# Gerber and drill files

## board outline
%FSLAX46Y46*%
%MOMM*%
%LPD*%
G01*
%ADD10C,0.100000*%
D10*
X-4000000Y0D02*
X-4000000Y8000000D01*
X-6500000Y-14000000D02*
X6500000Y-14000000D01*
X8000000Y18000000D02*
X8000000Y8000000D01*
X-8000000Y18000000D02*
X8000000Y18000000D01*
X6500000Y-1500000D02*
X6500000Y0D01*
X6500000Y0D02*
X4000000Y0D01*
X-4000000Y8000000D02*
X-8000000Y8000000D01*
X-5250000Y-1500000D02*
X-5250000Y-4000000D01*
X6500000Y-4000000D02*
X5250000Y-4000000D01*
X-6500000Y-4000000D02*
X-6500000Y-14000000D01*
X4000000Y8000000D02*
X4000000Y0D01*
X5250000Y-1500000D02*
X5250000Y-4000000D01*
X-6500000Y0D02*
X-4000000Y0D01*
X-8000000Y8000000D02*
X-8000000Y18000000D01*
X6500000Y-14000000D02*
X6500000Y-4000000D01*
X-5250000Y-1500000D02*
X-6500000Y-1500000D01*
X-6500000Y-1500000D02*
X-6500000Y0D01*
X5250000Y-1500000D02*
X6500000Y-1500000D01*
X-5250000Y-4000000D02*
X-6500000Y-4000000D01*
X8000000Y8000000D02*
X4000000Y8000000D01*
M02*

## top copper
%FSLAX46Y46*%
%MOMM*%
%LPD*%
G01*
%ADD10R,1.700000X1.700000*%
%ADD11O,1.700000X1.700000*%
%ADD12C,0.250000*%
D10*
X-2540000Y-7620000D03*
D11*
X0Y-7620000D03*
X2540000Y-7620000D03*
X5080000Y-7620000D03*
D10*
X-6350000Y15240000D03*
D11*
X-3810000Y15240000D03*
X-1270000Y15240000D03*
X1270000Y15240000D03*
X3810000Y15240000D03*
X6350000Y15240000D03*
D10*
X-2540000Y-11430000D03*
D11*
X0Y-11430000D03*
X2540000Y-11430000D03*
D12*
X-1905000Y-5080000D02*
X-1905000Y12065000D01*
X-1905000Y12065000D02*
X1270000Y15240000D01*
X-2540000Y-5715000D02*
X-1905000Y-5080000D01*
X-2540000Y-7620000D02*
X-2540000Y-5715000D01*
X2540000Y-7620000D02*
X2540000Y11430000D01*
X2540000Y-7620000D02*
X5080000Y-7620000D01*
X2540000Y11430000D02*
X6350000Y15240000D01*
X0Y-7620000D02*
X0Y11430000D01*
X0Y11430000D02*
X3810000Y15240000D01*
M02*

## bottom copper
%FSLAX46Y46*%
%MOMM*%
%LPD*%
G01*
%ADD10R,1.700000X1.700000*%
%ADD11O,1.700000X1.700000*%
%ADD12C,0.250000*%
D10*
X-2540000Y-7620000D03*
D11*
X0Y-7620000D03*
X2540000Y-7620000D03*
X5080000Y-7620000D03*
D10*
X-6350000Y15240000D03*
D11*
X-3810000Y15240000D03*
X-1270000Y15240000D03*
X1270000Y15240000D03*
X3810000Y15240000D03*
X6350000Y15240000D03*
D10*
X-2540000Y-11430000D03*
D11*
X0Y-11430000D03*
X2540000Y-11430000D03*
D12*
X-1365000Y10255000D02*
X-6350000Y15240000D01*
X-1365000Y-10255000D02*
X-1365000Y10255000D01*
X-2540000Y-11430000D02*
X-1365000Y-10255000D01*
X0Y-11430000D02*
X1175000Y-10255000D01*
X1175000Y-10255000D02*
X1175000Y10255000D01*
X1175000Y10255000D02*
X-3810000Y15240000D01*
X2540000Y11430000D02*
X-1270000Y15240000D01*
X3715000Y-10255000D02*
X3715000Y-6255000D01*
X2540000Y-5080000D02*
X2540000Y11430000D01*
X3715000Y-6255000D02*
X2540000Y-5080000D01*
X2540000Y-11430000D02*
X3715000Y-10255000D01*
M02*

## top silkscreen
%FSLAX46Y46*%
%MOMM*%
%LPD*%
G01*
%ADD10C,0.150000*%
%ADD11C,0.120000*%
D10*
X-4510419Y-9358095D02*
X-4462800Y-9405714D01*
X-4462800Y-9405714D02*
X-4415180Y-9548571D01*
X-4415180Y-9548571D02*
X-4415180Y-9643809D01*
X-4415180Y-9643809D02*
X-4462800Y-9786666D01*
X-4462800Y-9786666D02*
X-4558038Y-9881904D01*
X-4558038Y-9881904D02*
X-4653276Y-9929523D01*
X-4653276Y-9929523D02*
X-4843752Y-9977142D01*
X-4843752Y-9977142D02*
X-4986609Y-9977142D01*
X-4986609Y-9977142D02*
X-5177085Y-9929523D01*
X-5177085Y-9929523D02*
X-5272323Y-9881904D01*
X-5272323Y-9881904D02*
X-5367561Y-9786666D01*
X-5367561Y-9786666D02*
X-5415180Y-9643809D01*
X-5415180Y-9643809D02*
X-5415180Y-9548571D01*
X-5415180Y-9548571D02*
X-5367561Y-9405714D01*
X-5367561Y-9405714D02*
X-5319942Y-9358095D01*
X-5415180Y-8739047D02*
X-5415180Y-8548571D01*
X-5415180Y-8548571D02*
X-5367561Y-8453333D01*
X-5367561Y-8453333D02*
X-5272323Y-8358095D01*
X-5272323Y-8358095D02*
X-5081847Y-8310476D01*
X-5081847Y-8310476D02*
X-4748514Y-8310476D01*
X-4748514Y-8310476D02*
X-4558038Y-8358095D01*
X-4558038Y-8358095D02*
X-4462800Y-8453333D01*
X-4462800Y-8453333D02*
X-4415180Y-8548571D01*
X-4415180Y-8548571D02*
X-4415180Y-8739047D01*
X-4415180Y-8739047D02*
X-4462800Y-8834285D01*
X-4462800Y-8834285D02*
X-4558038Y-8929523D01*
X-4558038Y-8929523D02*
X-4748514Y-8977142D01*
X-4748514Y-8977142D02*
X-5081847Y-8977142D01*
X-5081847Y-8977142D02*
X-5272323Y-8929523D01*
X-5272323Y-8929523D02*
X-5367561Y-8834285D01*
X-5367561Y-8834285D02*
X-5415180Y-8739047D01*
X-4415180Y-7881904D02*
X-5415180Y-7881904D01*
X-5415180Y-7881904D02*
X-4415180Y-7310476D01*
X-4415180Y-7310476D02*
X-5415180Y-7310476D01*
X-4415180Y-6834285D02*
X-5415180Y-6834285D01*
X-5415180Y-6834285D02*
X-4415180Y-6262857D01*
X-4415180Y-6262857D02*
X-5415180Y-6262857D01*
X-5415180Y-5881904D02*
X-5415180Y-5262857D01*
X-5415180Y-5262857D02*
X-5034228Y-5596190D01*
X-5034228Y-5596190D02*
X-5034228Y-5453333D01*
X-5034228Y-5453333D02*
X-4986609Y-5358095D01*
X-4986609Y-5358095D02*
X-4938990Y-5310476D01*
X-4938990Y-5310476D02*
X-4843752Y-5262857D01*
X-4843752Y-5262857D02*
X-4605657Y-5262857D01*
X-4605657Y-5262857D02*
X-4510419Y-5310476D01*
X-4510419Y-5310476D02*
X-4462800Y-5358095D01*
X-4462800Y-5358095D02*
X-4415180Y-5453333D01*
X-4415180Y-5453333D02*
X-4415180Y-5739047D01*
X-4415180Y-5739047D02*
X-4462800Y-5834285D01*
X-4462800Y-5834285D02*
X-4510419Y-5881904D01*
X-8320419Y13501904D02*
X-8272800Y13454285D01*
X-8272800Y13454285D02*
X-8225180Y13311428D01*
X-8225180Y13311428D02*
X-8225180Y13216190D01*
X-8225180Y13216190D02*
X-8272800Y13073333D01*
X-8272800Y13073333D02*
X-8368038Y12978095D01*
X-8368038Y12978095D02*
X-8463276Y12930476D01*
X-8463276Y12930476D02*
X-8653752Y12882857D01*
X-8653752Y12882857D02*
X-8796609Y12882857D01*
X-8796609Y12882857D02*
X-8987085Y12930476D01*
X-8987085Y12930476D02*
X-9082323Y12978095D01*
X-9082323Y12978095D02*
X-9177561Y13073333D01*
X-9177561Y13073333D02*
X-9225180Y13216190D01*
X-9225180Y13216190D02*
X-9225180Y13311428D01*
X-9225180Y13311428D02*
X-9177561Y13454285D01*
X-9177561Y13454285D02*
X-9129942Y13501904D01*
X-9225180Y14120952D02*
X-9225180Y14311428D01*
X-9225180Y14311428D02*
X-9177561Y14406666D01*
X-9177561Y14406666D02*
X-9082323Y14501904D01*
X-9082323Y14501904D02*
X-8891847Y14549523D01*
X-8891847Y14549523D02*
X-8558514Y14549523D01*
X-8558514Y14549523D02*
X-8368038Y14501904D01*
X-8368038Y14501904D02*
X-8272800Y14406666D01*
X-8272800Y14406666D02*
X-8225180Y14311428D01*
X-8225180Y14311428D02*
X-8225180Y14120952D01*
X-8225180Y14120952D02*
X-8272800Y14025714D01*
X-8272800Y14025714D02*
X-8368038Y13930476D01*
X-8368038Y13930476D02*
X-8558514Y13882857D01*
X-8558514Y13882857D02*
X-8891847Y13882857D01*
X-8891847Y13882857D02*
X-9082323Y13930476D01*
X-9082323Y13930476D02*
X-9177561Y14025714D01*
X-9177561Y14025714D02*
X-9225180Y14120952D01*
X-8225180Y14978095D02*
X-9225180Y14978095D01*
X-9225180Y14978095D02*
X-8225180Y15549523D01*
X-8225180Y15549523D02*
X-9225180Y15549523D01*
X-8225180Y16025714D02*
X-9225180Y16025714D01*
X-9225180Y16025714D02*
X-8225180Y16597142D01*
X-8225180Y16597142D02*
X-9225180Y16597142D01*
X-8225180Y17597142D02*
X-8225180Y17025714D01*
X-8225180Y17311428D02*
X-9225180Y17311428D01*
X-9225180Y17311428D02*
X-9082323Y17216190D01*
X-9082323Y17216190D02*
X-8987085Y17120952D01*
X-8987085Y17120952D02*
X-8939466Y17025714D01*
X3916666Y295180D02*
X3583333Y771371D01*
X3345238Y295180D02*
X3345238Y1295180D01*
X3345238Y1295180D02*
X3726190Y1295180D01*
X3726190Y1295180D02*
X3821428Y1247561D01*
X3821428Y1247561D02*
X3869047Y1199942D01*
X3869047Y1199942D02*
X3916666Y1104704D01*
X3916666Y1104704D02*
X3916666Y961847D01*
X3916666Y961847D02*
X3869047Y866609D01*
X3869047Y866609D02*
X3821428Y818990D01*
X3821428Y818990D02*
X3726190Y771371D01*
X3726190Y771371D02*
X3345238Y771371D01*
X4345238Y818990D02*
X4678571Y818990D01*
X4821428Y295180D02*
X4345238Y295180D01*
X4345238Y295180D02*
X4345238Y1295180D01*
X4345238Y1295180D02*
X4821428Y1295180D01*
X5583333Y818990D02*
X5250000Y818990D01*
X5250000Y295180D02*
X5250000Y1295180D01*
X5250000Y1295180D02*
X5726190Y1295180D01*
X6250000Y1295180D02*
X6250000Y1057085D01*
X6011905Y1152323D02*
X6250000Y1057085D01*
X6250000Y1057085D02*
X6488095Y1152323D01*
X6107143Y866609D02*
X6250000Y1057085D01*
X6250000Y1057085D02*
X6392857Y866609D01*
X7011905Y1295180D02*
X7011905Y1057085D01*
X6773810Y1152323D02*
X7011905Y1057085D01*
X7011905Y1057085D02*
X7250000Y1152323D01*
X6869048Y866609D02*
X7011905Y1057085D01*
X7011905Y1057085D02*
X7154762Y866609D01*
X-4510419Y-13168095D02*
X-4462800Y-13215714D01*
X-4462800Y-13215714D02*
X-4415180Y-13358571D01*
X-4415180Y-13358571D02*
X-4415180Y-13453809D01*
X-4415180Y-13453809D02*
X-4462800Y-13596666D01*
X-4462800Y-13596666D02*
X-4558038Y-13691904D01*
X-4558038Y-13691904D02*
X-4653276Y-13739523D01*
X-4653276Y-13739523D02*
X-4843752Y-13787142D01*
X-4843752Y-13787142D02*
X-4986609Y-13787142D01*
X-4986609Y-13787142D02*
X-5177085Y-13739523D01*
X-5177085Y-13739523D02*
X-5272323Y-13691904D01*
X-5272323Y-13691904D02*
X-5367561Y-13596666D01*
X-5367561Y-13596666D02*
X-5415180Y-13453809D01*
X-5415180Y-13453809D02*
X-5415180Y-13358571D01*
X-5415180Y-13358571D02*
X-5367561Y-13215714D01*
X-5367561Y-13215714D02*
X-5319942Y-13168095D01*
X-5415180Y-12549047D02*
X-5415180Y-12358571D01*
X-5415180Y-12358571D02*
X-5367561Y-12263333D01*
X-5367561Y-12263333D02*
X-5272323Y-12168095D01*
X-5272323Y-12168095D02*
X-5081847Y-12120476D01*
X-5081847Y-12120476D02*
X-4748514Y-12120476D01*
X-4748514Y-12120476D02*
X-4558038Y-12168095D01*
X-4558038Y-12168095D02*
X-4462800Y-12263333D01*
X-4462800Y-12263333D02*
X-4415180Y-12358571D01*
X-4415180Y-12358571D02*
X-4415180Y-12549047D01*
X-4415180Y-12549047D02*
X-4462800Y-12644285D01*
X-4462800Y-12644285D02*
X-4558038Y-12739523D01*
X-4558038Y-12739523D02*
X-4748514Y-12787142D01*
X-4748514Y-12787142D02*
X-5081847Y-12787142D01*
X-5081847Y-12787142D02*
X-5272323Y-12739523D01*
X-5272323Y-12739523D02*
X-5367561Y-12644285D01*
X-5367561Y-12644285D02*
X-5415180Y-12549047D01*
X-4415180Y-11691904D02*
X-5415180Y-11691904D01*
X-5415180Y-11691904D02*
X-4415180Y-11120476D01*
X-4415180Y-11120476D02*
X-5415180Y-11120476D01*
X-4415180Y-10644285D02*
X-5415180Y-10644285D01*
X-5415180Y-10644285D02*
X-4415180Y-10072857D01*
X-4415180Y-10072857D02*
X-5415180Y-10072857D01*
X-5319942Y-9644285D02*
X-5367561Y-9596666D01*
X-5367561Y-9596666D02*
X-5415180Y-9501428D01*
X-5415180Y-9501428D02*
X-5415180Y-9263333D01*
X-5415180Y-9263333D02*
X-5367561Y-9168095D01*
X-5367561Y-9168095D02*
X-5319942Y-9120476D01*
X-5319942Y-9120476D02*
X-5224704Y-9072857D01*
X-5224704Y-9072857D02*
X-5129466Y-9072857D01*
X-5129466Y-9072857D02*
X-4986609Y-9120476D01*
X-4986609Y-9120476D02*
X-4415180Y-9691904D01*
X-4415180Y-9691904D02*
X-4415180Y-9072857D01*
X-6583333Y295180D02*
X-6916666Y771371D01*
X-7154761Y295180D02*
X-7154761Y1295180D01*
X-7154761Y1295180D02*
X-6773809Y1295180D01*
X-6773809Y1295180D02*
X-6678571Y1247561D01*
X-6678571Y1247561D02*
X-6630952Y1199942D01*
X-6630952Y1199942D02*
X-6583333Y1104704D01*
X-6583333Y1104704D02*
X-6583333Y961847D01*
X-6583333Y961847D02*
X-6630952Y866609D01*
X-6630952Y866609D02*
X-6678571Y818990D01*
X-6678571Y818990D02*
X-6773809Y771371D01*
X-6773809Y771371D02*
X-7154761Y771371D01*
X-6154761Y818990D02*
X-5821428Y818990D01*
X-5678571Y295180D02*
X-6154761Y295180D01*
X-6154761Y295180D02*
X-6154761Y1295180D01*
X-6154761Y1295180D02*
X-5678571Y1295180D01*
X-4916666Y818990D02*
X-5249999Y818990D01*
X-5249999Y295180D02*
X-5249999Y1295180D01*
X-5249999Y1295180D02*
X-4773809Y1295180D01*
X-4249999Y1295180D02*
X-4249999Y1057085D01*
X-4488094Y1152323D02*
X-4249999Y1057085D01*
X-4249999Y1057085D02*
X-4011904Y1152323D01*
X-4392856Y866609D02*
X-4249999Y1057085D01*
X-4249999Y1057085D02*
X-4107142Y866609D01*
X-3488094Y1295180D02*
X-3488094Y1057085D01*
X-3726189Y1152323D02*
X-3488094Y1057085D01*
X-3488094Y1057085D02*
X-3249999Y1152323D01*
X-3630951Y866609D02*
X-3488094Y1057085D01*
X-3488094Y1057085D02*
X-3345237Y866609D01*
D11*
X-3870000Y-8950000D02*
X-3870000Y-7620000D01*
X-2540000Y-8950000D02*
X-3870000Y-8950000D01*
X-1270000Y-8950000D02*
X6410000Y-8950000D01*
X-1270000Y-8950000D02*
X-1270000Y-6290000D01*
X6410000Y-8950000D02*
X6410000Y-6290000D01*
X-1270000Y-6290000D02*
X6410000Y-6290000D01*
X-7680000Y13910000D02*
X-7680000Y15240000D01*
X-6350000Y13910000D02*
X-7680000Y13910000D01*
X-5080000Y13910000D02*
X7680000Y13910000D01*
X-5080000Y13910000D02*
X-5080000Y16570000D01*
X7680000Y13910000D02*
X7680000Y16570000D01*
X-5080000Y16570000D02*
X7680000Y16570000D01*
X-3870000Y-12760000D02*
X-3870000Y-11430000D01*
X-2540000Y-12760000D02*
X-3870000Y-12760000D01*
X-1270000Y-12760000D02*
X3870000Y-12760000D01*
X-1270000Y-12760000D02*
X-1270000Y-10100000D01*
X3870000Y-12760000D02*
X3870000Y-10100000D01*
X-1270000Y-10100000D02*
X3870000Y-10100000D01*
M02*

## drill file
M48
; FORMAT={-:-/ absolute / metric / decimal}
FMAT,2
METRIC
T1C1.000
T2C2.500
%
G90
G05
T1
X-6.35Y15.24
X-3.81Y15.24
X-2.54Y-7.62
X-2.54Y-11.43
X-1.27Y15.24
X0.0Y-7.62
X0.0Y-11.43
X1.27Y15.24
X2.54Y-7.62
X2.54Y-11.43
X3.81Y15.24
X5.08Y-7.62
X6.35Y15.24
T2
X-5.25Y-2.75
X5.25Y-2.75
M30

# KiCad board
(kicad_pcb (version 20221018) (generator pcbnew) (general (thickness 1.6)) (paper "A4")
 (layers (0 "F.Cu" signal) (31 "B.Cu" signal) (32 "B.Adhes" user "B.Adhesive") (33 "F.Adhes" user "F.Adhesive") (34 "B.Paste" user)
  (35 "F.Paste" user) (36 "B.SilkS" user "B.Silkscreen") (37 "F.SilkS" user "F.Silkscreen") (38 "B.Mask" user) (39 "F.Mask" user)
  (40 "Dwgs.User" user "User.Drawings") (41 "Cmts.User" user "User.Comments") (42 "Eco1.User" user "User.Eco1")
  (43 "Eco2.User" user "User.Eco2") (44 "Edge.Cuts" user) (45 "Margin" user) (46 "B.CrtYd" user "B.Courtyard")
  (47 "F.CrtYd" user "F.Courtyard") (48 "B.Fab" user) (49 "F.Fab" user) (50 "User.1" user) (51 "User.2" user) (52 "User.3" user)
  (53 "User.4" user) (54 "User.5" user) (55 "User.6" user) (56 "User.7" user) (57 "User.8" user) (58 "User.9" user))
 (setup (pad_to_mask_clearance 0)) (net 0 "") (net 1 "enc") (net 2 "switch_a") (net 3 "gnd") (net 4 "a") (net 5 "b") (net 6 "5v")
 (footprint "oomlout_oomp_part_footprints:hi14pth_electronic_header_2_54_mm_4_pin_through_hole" (layer "F.Cu") (at -2.54 7.62 90)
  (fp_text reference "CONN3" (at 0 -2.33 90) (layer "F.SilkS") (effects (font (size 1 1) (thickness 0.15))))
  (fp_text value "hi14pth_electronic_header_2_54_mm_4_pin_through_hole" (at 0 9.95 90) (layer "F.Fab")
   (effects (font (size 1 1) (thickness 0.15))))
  (fp_line (start -1.33 -1.33) (end 0 -1.33) (stroke (width 0.12) (type solid)) (layer "F.SilkS"))
  (fp_line (start -1.33 0) (end -1.33 -1.33) (stroke (width 0.12) (type solid)) (layer "F.SilkS"))
  (fp_line (start -1.33 1.27) (end -1.33 8.95) (stroke (width 0.12) (type solid)) (layer "F.SilkS"))
  (fp_line (start -1.33 1.27) (end 1.33 1.27) (stroke (width 0.12) (type solid)) (layer "F.SilkS"))
  (fp_line (start -1.33 8.95) (end 1.33 8.95) (stroke (width 0.12) (type solid)) (layer "F.SilkS"))
  (fp_line (start 1.33 1.27) (end 1.33 8.95) (stroke (width 0.12) (type solid)) (layer "F.SilkS"))
  (pad "1" thru_hole rect (at 0 0 90) (size 1.7 1.7) (drill 1) (layers "*.Cu" "*.Mask") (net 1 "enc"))
  (pad "2" thru_hole oval (at 0 2.54 90) (size 1.7 1.7) (drill 1) (layers "*.Cu" "*.Mask") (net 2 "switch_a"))
  (pad "3" thru_hole oval (at 0 5.08 90) (size 1.7 1.7) (drill 1) (layers "*.Cu" "*.Mask") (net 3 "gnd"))
  (pad "4" thru_hole oval (at 0 7.62 90) (size 1.7 1.7) (drill 1) (layers "*.Cu" "*.Mask") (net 3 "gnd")))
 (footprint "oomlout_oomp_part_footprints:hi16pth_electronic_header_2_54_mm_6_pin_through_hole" (layer "F.Cu") (at -6.35 -15.24 90)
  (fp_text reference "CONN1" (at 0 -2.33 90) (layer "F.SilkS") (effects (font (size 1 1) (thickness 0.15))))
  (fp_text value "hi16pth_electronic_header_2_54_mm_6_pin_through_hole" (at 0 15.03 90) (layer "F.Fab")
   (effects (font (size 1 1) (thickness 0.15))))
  (fp_line (start -1.33 -1.33) (end 0 -1.33) (stroke (width 0.12) (type solid)) (layer "F.SilkS"))
  (fp_line (start -1.33 0) (end -1.33 -1.33) (stroke (width 0.12) (type solid)) (layer "F.SilkS"))
  (fp_line (start -1.33 1.27) (end -1.33 14.03) (stroke (width 0.12) (type solid)) (layer "F.SilkS"))
  (fp_line (start -1.33 1.27) (end 1.33 1.27) (stroke (width 0.12) (type solid)) (layer "F.SilkS"))
  (fp_line (start -1.33 14.03) (end 1.33 14.03) (stroke (width 0.12) (type solid)) (layer "F.SilkS"))
  (fp_line (start 1.33 1.27) (end 1.33 14.03) (stroke (width 0.12) (type solid)) (layer "F.SilkS"))
  (pad "1" thru_hole rect (at 0 0 90) (size 1.7 1.7) (drill 1) (layers "*.Cu" "*.Mask") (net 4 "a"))
  (pad "2" thru_hole oval (at 0 2.54 90) (size 1.7 1.7) (drill 1) (layers "*.Cu" "*.Mask") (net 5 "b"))
  (pad "3" thru_hole oval (at 0 5.08 90) (size 1.7 1.7) (drill 1) (layers "*.Cu" "*.Mask") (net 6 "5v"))
  (pad "4" thru_hole oval (at 0 7.62 90) (size 1.7 1.7) (drill 1) (layers "*.Cu" "*.Mask") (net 1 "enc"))
  (pad "5" thru_hole oval (at 0 10.16 90) (size 1.7 1.7) (drill 1) (layers "*.Cu" "*.Mask") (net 2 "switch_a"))
  (pad "6" thru_hole oval (at 0 12.7 90) (size 1.7 1.7) (drill 1) (layers "*.Cu" "*.Mask") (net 3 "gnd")))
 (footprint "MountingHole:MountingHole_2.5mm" (layer "F.Cu") (at 5.25 2.75)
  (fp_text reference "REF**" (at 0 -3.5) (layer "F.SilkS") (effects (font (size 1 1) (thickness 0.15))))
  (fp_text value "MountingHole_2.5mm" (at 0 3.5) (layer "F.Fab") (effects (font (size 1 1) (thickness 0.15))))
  (pad "" np_thru_hole circle (at 0 0) (size 2.5 2.5) (drill 2.5) (layers "*.Cu" "*.Mask")))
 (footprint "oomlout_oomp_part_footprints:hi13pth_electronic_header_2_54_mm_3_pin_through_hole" (layer "F.Cu") (at -2.54 11.43 90)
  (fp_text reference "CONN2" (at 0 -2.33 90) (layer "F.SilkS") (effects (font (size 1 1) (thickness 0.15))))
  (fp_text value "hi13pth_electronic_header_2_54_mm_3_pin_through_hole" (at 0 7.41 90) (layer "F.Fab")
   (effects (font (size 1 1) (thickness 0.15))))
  (fp_line (start -1.33 -1.33) (end 0 -1.33) (stroke (width 0.12) (type solid)) (layer "F.SilkS"))
  (fp_line (start -1.33 0) (end -1.33 -1.33) (stroke (width 0.12) (type solid)) (layer "F.SilkS"))
  (fp_line (start -1.33 1.27) (end -1.33 6.41) (stroke (width 0.12) (type solid)) (layer "F.SilkS"))
  (fp_line (start -1.33 1.27) (end 1.33 1.27) (stroke (width 0.12) (type solid)) (layer "F.SilkS"))
  (fp_line (start -1.33 6.41) (end 1.33 6.41) (stroke (width 0.12) (type solid)) (layer "F.SilkS"))
  (fp_line (start 1.33 1.27) (end 1.33 6.41) (stroke (width 0.12) (type solid)) (layer "F.SilkS"))
  (pad "1" thru_hole rect (at 0 0 90) (size 1.7 1.7) (drill 1) (layers "*.Cu" "*.Mask") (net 4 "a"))
  (pad "2" thru_hole oval (at 0 2.54 90) (size 1.7 1.7) (drill 1) (layers "*.Cu" "*.Mask") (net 5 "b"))
  (pad "3" thru_hole oval (at 0 5.08 90) (size 1.7 1.7) (drill 1) (layers "*.Cu" "*.Mask") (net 6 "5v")))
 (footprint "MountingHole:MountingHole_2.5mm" (layer "F.Cu") (at -5.25 2.75)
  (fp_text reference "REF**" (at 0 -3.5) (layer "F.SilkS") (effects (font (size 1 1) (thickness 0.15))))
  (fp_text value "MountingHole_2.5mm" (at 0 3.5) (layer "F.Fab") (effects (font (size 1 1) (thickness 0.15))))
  (pad "" np_thru_hole circle (at 0 0) (size 2.5 2.5) (drill 2.5) (layers "F&B.Cu" "*.Mask")))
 (gr_line (start -4 0) (end -4 -8) (stroke (width 0.1) (type default)) (layer "Edge.Cuts"))
 (gr_line (start -6.5 14) (end 6.5 14) (stroke (width 0.1) (type default)) (layer "Edge.Cuts"))
 (gr_line (start 8 -18) (end 8 -8) (stroke (width 0.1) (type default)) (layer "Edge.Cuts"))
 (gr_line (start -8 -18) (end 8 -18) (stroke (width 0.1) (type default)) (layer "Edge.Cuts"))
 (gr_line (start 6.5 1.5) (end 6.5 0) (stroke (width 0.1) (type default)) (layer "Edge.Cuts"))
 (gr_line (start 6.5 0) (end 4 0) (stroke (width 0.1) (type default)) (layer "Edge.Cuts"))
 (gr_line (start -4 -8) (end -8 -8) (stroke (width 0.1) (type default)) (layer "Edge.Cuts"))
 (gr_line (start -5.25 1.5) (end -5.25 4) (stroke (width 0.1) (type default)) (layer "Edge.Cuts"))
 (gr_line (start 6.5 4) (end 5.25 4) (stroke (width 0.1) (type default)) (layer "Edge.Cuts"))
 (gr_line (start -6.5 4) (end -6.5 14) (stroke (width 0.1) (type default)) (layer "Edge.Cuts"))
 (gr_line (start 4 -8) (end 4 0) (stroke (width 0.1) (type default)) (layer "Edge.Cuts"))
 (gr_line (start 5.25 1.5) (end 5.25 4) (stroke (width 0.1) (type default)) (layer "Edge.Cuts"))
 (gr_line (start -6.5 0) (end -4 0) (stroke (width 0.1) (type default)) (layer "Edge.Cuts"))
 (gr_line (start -8 -8) (end -8 -18) (stroke (width 0.1) (type default)) (layer "Edge.Cuts"))
 (gr_line (start 6.5 14) (end 6.5 4) (stroke (width 0.1) (type default)) (layer "Edge.Cuts"))
 (gr_line (start -5.25 1.5) (end -6.5 1.5) (stroke (width 0.1) (type default)) (layer "Edge.Cuts"))
 (gr_line (start -6.5 1.5) (end -6.5 0) (stroke (width 0.1) (type default)) (layer "Edge.Cuts"))
 (gr_line (start 5.25 1.5) (end 6.5 1.5) (stroke (width 0.1) (type default)) (layer "Edge.Cuts"))
 (gr_line (start -5.25 4) (end -6.5 4) (stroke (width 0.1) (type default)) (layer "Edge.Cuts"))
 (gr_line (start 8 -8) (end 4 -8) (stroke (width 0.1) (type default)) (layer "Edge.Cuts"))
 (segment (start -1.365 -10.255) (end -6.35 -15.24) (width 0.25) (layer "B.Cu") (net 4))
 (segment (start -1.365 10.255) (end -1.365 -10.255) (width 0.25) (layer "B.Cu") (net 4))
 (segment (start -2.54 11.43) (end -1.365 10.255) (width 0.25) (layer "B.Cu") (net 4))
 (segment (start 0 11.43) (end 1.175 10.255) (width 0.25) (layer "B.Cu") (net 5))
 (segment (start 1.175 10.255) (end 1.175 -10.255) (width 0.25) (layer "B.Cu") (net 5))
 (segment (start 1.175 -10.255) (end -3.81 -15.24) (width 0.25) (layer "B.Cu") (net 5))
 (segment (start 2.54 -11.43) (end -1.27 -15.24) (width 0.25) (layer "B.Cu") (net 6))
 (segment (start 3.715 10.255) (end 3.715 6.255) (width 0.25) (layer "B.Cu") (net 6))
 (segment (start 2.54 5.08) (end 2.54 -11.43) (width 0.25) (layer "B.Cu") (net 6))
 (segment (start 3.715 6.255) (end 2.54 5.08) (width 0.25) (layer "B.Cu") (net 6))
 (segment (start 2.54 11.43) (end 3.715 10.255) (width 0.25) (layer "B.Cu") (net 6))
 (segment (start -1.905 5.08) (end -1.905 -12.065) (width 0.25) (layer "F.Cu") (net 1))
 (segment (start -1.905 -12.065) (end 1.27 -15.24) (width 0.25) (layer "F.Cu") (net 1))
 (segment (start -2.54 5.715) (end -1.905 5.08) (width 0.25) (layer "F.Cu") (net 1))
 (segment (start -2.54 7.62) (end -2.54 5.715) (width 0.25) (layer "F.Cu") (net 1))
 (segment (start 2.54 7.62) (end 2.54 -11.43) (width 0.25) (layer "F.Cu") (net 3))
 (segment (start 2.54 7.62) (end 5.08 7.62) (width 0.25) (layer "F.Cu") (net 3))
 (segment (start 2.54 -11.43) (end 6.35 -15.24) (width 0.25) (layer "F.Cu") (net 3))
 (segment (start 0 7.62) (end 0 -11.43) (width 0.25) (layer "F.Cu") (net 2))
 (segment (start 0 -11.43) (end 3.81 -15.24) (width 0.25) (layer "F.Cu") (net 2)))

